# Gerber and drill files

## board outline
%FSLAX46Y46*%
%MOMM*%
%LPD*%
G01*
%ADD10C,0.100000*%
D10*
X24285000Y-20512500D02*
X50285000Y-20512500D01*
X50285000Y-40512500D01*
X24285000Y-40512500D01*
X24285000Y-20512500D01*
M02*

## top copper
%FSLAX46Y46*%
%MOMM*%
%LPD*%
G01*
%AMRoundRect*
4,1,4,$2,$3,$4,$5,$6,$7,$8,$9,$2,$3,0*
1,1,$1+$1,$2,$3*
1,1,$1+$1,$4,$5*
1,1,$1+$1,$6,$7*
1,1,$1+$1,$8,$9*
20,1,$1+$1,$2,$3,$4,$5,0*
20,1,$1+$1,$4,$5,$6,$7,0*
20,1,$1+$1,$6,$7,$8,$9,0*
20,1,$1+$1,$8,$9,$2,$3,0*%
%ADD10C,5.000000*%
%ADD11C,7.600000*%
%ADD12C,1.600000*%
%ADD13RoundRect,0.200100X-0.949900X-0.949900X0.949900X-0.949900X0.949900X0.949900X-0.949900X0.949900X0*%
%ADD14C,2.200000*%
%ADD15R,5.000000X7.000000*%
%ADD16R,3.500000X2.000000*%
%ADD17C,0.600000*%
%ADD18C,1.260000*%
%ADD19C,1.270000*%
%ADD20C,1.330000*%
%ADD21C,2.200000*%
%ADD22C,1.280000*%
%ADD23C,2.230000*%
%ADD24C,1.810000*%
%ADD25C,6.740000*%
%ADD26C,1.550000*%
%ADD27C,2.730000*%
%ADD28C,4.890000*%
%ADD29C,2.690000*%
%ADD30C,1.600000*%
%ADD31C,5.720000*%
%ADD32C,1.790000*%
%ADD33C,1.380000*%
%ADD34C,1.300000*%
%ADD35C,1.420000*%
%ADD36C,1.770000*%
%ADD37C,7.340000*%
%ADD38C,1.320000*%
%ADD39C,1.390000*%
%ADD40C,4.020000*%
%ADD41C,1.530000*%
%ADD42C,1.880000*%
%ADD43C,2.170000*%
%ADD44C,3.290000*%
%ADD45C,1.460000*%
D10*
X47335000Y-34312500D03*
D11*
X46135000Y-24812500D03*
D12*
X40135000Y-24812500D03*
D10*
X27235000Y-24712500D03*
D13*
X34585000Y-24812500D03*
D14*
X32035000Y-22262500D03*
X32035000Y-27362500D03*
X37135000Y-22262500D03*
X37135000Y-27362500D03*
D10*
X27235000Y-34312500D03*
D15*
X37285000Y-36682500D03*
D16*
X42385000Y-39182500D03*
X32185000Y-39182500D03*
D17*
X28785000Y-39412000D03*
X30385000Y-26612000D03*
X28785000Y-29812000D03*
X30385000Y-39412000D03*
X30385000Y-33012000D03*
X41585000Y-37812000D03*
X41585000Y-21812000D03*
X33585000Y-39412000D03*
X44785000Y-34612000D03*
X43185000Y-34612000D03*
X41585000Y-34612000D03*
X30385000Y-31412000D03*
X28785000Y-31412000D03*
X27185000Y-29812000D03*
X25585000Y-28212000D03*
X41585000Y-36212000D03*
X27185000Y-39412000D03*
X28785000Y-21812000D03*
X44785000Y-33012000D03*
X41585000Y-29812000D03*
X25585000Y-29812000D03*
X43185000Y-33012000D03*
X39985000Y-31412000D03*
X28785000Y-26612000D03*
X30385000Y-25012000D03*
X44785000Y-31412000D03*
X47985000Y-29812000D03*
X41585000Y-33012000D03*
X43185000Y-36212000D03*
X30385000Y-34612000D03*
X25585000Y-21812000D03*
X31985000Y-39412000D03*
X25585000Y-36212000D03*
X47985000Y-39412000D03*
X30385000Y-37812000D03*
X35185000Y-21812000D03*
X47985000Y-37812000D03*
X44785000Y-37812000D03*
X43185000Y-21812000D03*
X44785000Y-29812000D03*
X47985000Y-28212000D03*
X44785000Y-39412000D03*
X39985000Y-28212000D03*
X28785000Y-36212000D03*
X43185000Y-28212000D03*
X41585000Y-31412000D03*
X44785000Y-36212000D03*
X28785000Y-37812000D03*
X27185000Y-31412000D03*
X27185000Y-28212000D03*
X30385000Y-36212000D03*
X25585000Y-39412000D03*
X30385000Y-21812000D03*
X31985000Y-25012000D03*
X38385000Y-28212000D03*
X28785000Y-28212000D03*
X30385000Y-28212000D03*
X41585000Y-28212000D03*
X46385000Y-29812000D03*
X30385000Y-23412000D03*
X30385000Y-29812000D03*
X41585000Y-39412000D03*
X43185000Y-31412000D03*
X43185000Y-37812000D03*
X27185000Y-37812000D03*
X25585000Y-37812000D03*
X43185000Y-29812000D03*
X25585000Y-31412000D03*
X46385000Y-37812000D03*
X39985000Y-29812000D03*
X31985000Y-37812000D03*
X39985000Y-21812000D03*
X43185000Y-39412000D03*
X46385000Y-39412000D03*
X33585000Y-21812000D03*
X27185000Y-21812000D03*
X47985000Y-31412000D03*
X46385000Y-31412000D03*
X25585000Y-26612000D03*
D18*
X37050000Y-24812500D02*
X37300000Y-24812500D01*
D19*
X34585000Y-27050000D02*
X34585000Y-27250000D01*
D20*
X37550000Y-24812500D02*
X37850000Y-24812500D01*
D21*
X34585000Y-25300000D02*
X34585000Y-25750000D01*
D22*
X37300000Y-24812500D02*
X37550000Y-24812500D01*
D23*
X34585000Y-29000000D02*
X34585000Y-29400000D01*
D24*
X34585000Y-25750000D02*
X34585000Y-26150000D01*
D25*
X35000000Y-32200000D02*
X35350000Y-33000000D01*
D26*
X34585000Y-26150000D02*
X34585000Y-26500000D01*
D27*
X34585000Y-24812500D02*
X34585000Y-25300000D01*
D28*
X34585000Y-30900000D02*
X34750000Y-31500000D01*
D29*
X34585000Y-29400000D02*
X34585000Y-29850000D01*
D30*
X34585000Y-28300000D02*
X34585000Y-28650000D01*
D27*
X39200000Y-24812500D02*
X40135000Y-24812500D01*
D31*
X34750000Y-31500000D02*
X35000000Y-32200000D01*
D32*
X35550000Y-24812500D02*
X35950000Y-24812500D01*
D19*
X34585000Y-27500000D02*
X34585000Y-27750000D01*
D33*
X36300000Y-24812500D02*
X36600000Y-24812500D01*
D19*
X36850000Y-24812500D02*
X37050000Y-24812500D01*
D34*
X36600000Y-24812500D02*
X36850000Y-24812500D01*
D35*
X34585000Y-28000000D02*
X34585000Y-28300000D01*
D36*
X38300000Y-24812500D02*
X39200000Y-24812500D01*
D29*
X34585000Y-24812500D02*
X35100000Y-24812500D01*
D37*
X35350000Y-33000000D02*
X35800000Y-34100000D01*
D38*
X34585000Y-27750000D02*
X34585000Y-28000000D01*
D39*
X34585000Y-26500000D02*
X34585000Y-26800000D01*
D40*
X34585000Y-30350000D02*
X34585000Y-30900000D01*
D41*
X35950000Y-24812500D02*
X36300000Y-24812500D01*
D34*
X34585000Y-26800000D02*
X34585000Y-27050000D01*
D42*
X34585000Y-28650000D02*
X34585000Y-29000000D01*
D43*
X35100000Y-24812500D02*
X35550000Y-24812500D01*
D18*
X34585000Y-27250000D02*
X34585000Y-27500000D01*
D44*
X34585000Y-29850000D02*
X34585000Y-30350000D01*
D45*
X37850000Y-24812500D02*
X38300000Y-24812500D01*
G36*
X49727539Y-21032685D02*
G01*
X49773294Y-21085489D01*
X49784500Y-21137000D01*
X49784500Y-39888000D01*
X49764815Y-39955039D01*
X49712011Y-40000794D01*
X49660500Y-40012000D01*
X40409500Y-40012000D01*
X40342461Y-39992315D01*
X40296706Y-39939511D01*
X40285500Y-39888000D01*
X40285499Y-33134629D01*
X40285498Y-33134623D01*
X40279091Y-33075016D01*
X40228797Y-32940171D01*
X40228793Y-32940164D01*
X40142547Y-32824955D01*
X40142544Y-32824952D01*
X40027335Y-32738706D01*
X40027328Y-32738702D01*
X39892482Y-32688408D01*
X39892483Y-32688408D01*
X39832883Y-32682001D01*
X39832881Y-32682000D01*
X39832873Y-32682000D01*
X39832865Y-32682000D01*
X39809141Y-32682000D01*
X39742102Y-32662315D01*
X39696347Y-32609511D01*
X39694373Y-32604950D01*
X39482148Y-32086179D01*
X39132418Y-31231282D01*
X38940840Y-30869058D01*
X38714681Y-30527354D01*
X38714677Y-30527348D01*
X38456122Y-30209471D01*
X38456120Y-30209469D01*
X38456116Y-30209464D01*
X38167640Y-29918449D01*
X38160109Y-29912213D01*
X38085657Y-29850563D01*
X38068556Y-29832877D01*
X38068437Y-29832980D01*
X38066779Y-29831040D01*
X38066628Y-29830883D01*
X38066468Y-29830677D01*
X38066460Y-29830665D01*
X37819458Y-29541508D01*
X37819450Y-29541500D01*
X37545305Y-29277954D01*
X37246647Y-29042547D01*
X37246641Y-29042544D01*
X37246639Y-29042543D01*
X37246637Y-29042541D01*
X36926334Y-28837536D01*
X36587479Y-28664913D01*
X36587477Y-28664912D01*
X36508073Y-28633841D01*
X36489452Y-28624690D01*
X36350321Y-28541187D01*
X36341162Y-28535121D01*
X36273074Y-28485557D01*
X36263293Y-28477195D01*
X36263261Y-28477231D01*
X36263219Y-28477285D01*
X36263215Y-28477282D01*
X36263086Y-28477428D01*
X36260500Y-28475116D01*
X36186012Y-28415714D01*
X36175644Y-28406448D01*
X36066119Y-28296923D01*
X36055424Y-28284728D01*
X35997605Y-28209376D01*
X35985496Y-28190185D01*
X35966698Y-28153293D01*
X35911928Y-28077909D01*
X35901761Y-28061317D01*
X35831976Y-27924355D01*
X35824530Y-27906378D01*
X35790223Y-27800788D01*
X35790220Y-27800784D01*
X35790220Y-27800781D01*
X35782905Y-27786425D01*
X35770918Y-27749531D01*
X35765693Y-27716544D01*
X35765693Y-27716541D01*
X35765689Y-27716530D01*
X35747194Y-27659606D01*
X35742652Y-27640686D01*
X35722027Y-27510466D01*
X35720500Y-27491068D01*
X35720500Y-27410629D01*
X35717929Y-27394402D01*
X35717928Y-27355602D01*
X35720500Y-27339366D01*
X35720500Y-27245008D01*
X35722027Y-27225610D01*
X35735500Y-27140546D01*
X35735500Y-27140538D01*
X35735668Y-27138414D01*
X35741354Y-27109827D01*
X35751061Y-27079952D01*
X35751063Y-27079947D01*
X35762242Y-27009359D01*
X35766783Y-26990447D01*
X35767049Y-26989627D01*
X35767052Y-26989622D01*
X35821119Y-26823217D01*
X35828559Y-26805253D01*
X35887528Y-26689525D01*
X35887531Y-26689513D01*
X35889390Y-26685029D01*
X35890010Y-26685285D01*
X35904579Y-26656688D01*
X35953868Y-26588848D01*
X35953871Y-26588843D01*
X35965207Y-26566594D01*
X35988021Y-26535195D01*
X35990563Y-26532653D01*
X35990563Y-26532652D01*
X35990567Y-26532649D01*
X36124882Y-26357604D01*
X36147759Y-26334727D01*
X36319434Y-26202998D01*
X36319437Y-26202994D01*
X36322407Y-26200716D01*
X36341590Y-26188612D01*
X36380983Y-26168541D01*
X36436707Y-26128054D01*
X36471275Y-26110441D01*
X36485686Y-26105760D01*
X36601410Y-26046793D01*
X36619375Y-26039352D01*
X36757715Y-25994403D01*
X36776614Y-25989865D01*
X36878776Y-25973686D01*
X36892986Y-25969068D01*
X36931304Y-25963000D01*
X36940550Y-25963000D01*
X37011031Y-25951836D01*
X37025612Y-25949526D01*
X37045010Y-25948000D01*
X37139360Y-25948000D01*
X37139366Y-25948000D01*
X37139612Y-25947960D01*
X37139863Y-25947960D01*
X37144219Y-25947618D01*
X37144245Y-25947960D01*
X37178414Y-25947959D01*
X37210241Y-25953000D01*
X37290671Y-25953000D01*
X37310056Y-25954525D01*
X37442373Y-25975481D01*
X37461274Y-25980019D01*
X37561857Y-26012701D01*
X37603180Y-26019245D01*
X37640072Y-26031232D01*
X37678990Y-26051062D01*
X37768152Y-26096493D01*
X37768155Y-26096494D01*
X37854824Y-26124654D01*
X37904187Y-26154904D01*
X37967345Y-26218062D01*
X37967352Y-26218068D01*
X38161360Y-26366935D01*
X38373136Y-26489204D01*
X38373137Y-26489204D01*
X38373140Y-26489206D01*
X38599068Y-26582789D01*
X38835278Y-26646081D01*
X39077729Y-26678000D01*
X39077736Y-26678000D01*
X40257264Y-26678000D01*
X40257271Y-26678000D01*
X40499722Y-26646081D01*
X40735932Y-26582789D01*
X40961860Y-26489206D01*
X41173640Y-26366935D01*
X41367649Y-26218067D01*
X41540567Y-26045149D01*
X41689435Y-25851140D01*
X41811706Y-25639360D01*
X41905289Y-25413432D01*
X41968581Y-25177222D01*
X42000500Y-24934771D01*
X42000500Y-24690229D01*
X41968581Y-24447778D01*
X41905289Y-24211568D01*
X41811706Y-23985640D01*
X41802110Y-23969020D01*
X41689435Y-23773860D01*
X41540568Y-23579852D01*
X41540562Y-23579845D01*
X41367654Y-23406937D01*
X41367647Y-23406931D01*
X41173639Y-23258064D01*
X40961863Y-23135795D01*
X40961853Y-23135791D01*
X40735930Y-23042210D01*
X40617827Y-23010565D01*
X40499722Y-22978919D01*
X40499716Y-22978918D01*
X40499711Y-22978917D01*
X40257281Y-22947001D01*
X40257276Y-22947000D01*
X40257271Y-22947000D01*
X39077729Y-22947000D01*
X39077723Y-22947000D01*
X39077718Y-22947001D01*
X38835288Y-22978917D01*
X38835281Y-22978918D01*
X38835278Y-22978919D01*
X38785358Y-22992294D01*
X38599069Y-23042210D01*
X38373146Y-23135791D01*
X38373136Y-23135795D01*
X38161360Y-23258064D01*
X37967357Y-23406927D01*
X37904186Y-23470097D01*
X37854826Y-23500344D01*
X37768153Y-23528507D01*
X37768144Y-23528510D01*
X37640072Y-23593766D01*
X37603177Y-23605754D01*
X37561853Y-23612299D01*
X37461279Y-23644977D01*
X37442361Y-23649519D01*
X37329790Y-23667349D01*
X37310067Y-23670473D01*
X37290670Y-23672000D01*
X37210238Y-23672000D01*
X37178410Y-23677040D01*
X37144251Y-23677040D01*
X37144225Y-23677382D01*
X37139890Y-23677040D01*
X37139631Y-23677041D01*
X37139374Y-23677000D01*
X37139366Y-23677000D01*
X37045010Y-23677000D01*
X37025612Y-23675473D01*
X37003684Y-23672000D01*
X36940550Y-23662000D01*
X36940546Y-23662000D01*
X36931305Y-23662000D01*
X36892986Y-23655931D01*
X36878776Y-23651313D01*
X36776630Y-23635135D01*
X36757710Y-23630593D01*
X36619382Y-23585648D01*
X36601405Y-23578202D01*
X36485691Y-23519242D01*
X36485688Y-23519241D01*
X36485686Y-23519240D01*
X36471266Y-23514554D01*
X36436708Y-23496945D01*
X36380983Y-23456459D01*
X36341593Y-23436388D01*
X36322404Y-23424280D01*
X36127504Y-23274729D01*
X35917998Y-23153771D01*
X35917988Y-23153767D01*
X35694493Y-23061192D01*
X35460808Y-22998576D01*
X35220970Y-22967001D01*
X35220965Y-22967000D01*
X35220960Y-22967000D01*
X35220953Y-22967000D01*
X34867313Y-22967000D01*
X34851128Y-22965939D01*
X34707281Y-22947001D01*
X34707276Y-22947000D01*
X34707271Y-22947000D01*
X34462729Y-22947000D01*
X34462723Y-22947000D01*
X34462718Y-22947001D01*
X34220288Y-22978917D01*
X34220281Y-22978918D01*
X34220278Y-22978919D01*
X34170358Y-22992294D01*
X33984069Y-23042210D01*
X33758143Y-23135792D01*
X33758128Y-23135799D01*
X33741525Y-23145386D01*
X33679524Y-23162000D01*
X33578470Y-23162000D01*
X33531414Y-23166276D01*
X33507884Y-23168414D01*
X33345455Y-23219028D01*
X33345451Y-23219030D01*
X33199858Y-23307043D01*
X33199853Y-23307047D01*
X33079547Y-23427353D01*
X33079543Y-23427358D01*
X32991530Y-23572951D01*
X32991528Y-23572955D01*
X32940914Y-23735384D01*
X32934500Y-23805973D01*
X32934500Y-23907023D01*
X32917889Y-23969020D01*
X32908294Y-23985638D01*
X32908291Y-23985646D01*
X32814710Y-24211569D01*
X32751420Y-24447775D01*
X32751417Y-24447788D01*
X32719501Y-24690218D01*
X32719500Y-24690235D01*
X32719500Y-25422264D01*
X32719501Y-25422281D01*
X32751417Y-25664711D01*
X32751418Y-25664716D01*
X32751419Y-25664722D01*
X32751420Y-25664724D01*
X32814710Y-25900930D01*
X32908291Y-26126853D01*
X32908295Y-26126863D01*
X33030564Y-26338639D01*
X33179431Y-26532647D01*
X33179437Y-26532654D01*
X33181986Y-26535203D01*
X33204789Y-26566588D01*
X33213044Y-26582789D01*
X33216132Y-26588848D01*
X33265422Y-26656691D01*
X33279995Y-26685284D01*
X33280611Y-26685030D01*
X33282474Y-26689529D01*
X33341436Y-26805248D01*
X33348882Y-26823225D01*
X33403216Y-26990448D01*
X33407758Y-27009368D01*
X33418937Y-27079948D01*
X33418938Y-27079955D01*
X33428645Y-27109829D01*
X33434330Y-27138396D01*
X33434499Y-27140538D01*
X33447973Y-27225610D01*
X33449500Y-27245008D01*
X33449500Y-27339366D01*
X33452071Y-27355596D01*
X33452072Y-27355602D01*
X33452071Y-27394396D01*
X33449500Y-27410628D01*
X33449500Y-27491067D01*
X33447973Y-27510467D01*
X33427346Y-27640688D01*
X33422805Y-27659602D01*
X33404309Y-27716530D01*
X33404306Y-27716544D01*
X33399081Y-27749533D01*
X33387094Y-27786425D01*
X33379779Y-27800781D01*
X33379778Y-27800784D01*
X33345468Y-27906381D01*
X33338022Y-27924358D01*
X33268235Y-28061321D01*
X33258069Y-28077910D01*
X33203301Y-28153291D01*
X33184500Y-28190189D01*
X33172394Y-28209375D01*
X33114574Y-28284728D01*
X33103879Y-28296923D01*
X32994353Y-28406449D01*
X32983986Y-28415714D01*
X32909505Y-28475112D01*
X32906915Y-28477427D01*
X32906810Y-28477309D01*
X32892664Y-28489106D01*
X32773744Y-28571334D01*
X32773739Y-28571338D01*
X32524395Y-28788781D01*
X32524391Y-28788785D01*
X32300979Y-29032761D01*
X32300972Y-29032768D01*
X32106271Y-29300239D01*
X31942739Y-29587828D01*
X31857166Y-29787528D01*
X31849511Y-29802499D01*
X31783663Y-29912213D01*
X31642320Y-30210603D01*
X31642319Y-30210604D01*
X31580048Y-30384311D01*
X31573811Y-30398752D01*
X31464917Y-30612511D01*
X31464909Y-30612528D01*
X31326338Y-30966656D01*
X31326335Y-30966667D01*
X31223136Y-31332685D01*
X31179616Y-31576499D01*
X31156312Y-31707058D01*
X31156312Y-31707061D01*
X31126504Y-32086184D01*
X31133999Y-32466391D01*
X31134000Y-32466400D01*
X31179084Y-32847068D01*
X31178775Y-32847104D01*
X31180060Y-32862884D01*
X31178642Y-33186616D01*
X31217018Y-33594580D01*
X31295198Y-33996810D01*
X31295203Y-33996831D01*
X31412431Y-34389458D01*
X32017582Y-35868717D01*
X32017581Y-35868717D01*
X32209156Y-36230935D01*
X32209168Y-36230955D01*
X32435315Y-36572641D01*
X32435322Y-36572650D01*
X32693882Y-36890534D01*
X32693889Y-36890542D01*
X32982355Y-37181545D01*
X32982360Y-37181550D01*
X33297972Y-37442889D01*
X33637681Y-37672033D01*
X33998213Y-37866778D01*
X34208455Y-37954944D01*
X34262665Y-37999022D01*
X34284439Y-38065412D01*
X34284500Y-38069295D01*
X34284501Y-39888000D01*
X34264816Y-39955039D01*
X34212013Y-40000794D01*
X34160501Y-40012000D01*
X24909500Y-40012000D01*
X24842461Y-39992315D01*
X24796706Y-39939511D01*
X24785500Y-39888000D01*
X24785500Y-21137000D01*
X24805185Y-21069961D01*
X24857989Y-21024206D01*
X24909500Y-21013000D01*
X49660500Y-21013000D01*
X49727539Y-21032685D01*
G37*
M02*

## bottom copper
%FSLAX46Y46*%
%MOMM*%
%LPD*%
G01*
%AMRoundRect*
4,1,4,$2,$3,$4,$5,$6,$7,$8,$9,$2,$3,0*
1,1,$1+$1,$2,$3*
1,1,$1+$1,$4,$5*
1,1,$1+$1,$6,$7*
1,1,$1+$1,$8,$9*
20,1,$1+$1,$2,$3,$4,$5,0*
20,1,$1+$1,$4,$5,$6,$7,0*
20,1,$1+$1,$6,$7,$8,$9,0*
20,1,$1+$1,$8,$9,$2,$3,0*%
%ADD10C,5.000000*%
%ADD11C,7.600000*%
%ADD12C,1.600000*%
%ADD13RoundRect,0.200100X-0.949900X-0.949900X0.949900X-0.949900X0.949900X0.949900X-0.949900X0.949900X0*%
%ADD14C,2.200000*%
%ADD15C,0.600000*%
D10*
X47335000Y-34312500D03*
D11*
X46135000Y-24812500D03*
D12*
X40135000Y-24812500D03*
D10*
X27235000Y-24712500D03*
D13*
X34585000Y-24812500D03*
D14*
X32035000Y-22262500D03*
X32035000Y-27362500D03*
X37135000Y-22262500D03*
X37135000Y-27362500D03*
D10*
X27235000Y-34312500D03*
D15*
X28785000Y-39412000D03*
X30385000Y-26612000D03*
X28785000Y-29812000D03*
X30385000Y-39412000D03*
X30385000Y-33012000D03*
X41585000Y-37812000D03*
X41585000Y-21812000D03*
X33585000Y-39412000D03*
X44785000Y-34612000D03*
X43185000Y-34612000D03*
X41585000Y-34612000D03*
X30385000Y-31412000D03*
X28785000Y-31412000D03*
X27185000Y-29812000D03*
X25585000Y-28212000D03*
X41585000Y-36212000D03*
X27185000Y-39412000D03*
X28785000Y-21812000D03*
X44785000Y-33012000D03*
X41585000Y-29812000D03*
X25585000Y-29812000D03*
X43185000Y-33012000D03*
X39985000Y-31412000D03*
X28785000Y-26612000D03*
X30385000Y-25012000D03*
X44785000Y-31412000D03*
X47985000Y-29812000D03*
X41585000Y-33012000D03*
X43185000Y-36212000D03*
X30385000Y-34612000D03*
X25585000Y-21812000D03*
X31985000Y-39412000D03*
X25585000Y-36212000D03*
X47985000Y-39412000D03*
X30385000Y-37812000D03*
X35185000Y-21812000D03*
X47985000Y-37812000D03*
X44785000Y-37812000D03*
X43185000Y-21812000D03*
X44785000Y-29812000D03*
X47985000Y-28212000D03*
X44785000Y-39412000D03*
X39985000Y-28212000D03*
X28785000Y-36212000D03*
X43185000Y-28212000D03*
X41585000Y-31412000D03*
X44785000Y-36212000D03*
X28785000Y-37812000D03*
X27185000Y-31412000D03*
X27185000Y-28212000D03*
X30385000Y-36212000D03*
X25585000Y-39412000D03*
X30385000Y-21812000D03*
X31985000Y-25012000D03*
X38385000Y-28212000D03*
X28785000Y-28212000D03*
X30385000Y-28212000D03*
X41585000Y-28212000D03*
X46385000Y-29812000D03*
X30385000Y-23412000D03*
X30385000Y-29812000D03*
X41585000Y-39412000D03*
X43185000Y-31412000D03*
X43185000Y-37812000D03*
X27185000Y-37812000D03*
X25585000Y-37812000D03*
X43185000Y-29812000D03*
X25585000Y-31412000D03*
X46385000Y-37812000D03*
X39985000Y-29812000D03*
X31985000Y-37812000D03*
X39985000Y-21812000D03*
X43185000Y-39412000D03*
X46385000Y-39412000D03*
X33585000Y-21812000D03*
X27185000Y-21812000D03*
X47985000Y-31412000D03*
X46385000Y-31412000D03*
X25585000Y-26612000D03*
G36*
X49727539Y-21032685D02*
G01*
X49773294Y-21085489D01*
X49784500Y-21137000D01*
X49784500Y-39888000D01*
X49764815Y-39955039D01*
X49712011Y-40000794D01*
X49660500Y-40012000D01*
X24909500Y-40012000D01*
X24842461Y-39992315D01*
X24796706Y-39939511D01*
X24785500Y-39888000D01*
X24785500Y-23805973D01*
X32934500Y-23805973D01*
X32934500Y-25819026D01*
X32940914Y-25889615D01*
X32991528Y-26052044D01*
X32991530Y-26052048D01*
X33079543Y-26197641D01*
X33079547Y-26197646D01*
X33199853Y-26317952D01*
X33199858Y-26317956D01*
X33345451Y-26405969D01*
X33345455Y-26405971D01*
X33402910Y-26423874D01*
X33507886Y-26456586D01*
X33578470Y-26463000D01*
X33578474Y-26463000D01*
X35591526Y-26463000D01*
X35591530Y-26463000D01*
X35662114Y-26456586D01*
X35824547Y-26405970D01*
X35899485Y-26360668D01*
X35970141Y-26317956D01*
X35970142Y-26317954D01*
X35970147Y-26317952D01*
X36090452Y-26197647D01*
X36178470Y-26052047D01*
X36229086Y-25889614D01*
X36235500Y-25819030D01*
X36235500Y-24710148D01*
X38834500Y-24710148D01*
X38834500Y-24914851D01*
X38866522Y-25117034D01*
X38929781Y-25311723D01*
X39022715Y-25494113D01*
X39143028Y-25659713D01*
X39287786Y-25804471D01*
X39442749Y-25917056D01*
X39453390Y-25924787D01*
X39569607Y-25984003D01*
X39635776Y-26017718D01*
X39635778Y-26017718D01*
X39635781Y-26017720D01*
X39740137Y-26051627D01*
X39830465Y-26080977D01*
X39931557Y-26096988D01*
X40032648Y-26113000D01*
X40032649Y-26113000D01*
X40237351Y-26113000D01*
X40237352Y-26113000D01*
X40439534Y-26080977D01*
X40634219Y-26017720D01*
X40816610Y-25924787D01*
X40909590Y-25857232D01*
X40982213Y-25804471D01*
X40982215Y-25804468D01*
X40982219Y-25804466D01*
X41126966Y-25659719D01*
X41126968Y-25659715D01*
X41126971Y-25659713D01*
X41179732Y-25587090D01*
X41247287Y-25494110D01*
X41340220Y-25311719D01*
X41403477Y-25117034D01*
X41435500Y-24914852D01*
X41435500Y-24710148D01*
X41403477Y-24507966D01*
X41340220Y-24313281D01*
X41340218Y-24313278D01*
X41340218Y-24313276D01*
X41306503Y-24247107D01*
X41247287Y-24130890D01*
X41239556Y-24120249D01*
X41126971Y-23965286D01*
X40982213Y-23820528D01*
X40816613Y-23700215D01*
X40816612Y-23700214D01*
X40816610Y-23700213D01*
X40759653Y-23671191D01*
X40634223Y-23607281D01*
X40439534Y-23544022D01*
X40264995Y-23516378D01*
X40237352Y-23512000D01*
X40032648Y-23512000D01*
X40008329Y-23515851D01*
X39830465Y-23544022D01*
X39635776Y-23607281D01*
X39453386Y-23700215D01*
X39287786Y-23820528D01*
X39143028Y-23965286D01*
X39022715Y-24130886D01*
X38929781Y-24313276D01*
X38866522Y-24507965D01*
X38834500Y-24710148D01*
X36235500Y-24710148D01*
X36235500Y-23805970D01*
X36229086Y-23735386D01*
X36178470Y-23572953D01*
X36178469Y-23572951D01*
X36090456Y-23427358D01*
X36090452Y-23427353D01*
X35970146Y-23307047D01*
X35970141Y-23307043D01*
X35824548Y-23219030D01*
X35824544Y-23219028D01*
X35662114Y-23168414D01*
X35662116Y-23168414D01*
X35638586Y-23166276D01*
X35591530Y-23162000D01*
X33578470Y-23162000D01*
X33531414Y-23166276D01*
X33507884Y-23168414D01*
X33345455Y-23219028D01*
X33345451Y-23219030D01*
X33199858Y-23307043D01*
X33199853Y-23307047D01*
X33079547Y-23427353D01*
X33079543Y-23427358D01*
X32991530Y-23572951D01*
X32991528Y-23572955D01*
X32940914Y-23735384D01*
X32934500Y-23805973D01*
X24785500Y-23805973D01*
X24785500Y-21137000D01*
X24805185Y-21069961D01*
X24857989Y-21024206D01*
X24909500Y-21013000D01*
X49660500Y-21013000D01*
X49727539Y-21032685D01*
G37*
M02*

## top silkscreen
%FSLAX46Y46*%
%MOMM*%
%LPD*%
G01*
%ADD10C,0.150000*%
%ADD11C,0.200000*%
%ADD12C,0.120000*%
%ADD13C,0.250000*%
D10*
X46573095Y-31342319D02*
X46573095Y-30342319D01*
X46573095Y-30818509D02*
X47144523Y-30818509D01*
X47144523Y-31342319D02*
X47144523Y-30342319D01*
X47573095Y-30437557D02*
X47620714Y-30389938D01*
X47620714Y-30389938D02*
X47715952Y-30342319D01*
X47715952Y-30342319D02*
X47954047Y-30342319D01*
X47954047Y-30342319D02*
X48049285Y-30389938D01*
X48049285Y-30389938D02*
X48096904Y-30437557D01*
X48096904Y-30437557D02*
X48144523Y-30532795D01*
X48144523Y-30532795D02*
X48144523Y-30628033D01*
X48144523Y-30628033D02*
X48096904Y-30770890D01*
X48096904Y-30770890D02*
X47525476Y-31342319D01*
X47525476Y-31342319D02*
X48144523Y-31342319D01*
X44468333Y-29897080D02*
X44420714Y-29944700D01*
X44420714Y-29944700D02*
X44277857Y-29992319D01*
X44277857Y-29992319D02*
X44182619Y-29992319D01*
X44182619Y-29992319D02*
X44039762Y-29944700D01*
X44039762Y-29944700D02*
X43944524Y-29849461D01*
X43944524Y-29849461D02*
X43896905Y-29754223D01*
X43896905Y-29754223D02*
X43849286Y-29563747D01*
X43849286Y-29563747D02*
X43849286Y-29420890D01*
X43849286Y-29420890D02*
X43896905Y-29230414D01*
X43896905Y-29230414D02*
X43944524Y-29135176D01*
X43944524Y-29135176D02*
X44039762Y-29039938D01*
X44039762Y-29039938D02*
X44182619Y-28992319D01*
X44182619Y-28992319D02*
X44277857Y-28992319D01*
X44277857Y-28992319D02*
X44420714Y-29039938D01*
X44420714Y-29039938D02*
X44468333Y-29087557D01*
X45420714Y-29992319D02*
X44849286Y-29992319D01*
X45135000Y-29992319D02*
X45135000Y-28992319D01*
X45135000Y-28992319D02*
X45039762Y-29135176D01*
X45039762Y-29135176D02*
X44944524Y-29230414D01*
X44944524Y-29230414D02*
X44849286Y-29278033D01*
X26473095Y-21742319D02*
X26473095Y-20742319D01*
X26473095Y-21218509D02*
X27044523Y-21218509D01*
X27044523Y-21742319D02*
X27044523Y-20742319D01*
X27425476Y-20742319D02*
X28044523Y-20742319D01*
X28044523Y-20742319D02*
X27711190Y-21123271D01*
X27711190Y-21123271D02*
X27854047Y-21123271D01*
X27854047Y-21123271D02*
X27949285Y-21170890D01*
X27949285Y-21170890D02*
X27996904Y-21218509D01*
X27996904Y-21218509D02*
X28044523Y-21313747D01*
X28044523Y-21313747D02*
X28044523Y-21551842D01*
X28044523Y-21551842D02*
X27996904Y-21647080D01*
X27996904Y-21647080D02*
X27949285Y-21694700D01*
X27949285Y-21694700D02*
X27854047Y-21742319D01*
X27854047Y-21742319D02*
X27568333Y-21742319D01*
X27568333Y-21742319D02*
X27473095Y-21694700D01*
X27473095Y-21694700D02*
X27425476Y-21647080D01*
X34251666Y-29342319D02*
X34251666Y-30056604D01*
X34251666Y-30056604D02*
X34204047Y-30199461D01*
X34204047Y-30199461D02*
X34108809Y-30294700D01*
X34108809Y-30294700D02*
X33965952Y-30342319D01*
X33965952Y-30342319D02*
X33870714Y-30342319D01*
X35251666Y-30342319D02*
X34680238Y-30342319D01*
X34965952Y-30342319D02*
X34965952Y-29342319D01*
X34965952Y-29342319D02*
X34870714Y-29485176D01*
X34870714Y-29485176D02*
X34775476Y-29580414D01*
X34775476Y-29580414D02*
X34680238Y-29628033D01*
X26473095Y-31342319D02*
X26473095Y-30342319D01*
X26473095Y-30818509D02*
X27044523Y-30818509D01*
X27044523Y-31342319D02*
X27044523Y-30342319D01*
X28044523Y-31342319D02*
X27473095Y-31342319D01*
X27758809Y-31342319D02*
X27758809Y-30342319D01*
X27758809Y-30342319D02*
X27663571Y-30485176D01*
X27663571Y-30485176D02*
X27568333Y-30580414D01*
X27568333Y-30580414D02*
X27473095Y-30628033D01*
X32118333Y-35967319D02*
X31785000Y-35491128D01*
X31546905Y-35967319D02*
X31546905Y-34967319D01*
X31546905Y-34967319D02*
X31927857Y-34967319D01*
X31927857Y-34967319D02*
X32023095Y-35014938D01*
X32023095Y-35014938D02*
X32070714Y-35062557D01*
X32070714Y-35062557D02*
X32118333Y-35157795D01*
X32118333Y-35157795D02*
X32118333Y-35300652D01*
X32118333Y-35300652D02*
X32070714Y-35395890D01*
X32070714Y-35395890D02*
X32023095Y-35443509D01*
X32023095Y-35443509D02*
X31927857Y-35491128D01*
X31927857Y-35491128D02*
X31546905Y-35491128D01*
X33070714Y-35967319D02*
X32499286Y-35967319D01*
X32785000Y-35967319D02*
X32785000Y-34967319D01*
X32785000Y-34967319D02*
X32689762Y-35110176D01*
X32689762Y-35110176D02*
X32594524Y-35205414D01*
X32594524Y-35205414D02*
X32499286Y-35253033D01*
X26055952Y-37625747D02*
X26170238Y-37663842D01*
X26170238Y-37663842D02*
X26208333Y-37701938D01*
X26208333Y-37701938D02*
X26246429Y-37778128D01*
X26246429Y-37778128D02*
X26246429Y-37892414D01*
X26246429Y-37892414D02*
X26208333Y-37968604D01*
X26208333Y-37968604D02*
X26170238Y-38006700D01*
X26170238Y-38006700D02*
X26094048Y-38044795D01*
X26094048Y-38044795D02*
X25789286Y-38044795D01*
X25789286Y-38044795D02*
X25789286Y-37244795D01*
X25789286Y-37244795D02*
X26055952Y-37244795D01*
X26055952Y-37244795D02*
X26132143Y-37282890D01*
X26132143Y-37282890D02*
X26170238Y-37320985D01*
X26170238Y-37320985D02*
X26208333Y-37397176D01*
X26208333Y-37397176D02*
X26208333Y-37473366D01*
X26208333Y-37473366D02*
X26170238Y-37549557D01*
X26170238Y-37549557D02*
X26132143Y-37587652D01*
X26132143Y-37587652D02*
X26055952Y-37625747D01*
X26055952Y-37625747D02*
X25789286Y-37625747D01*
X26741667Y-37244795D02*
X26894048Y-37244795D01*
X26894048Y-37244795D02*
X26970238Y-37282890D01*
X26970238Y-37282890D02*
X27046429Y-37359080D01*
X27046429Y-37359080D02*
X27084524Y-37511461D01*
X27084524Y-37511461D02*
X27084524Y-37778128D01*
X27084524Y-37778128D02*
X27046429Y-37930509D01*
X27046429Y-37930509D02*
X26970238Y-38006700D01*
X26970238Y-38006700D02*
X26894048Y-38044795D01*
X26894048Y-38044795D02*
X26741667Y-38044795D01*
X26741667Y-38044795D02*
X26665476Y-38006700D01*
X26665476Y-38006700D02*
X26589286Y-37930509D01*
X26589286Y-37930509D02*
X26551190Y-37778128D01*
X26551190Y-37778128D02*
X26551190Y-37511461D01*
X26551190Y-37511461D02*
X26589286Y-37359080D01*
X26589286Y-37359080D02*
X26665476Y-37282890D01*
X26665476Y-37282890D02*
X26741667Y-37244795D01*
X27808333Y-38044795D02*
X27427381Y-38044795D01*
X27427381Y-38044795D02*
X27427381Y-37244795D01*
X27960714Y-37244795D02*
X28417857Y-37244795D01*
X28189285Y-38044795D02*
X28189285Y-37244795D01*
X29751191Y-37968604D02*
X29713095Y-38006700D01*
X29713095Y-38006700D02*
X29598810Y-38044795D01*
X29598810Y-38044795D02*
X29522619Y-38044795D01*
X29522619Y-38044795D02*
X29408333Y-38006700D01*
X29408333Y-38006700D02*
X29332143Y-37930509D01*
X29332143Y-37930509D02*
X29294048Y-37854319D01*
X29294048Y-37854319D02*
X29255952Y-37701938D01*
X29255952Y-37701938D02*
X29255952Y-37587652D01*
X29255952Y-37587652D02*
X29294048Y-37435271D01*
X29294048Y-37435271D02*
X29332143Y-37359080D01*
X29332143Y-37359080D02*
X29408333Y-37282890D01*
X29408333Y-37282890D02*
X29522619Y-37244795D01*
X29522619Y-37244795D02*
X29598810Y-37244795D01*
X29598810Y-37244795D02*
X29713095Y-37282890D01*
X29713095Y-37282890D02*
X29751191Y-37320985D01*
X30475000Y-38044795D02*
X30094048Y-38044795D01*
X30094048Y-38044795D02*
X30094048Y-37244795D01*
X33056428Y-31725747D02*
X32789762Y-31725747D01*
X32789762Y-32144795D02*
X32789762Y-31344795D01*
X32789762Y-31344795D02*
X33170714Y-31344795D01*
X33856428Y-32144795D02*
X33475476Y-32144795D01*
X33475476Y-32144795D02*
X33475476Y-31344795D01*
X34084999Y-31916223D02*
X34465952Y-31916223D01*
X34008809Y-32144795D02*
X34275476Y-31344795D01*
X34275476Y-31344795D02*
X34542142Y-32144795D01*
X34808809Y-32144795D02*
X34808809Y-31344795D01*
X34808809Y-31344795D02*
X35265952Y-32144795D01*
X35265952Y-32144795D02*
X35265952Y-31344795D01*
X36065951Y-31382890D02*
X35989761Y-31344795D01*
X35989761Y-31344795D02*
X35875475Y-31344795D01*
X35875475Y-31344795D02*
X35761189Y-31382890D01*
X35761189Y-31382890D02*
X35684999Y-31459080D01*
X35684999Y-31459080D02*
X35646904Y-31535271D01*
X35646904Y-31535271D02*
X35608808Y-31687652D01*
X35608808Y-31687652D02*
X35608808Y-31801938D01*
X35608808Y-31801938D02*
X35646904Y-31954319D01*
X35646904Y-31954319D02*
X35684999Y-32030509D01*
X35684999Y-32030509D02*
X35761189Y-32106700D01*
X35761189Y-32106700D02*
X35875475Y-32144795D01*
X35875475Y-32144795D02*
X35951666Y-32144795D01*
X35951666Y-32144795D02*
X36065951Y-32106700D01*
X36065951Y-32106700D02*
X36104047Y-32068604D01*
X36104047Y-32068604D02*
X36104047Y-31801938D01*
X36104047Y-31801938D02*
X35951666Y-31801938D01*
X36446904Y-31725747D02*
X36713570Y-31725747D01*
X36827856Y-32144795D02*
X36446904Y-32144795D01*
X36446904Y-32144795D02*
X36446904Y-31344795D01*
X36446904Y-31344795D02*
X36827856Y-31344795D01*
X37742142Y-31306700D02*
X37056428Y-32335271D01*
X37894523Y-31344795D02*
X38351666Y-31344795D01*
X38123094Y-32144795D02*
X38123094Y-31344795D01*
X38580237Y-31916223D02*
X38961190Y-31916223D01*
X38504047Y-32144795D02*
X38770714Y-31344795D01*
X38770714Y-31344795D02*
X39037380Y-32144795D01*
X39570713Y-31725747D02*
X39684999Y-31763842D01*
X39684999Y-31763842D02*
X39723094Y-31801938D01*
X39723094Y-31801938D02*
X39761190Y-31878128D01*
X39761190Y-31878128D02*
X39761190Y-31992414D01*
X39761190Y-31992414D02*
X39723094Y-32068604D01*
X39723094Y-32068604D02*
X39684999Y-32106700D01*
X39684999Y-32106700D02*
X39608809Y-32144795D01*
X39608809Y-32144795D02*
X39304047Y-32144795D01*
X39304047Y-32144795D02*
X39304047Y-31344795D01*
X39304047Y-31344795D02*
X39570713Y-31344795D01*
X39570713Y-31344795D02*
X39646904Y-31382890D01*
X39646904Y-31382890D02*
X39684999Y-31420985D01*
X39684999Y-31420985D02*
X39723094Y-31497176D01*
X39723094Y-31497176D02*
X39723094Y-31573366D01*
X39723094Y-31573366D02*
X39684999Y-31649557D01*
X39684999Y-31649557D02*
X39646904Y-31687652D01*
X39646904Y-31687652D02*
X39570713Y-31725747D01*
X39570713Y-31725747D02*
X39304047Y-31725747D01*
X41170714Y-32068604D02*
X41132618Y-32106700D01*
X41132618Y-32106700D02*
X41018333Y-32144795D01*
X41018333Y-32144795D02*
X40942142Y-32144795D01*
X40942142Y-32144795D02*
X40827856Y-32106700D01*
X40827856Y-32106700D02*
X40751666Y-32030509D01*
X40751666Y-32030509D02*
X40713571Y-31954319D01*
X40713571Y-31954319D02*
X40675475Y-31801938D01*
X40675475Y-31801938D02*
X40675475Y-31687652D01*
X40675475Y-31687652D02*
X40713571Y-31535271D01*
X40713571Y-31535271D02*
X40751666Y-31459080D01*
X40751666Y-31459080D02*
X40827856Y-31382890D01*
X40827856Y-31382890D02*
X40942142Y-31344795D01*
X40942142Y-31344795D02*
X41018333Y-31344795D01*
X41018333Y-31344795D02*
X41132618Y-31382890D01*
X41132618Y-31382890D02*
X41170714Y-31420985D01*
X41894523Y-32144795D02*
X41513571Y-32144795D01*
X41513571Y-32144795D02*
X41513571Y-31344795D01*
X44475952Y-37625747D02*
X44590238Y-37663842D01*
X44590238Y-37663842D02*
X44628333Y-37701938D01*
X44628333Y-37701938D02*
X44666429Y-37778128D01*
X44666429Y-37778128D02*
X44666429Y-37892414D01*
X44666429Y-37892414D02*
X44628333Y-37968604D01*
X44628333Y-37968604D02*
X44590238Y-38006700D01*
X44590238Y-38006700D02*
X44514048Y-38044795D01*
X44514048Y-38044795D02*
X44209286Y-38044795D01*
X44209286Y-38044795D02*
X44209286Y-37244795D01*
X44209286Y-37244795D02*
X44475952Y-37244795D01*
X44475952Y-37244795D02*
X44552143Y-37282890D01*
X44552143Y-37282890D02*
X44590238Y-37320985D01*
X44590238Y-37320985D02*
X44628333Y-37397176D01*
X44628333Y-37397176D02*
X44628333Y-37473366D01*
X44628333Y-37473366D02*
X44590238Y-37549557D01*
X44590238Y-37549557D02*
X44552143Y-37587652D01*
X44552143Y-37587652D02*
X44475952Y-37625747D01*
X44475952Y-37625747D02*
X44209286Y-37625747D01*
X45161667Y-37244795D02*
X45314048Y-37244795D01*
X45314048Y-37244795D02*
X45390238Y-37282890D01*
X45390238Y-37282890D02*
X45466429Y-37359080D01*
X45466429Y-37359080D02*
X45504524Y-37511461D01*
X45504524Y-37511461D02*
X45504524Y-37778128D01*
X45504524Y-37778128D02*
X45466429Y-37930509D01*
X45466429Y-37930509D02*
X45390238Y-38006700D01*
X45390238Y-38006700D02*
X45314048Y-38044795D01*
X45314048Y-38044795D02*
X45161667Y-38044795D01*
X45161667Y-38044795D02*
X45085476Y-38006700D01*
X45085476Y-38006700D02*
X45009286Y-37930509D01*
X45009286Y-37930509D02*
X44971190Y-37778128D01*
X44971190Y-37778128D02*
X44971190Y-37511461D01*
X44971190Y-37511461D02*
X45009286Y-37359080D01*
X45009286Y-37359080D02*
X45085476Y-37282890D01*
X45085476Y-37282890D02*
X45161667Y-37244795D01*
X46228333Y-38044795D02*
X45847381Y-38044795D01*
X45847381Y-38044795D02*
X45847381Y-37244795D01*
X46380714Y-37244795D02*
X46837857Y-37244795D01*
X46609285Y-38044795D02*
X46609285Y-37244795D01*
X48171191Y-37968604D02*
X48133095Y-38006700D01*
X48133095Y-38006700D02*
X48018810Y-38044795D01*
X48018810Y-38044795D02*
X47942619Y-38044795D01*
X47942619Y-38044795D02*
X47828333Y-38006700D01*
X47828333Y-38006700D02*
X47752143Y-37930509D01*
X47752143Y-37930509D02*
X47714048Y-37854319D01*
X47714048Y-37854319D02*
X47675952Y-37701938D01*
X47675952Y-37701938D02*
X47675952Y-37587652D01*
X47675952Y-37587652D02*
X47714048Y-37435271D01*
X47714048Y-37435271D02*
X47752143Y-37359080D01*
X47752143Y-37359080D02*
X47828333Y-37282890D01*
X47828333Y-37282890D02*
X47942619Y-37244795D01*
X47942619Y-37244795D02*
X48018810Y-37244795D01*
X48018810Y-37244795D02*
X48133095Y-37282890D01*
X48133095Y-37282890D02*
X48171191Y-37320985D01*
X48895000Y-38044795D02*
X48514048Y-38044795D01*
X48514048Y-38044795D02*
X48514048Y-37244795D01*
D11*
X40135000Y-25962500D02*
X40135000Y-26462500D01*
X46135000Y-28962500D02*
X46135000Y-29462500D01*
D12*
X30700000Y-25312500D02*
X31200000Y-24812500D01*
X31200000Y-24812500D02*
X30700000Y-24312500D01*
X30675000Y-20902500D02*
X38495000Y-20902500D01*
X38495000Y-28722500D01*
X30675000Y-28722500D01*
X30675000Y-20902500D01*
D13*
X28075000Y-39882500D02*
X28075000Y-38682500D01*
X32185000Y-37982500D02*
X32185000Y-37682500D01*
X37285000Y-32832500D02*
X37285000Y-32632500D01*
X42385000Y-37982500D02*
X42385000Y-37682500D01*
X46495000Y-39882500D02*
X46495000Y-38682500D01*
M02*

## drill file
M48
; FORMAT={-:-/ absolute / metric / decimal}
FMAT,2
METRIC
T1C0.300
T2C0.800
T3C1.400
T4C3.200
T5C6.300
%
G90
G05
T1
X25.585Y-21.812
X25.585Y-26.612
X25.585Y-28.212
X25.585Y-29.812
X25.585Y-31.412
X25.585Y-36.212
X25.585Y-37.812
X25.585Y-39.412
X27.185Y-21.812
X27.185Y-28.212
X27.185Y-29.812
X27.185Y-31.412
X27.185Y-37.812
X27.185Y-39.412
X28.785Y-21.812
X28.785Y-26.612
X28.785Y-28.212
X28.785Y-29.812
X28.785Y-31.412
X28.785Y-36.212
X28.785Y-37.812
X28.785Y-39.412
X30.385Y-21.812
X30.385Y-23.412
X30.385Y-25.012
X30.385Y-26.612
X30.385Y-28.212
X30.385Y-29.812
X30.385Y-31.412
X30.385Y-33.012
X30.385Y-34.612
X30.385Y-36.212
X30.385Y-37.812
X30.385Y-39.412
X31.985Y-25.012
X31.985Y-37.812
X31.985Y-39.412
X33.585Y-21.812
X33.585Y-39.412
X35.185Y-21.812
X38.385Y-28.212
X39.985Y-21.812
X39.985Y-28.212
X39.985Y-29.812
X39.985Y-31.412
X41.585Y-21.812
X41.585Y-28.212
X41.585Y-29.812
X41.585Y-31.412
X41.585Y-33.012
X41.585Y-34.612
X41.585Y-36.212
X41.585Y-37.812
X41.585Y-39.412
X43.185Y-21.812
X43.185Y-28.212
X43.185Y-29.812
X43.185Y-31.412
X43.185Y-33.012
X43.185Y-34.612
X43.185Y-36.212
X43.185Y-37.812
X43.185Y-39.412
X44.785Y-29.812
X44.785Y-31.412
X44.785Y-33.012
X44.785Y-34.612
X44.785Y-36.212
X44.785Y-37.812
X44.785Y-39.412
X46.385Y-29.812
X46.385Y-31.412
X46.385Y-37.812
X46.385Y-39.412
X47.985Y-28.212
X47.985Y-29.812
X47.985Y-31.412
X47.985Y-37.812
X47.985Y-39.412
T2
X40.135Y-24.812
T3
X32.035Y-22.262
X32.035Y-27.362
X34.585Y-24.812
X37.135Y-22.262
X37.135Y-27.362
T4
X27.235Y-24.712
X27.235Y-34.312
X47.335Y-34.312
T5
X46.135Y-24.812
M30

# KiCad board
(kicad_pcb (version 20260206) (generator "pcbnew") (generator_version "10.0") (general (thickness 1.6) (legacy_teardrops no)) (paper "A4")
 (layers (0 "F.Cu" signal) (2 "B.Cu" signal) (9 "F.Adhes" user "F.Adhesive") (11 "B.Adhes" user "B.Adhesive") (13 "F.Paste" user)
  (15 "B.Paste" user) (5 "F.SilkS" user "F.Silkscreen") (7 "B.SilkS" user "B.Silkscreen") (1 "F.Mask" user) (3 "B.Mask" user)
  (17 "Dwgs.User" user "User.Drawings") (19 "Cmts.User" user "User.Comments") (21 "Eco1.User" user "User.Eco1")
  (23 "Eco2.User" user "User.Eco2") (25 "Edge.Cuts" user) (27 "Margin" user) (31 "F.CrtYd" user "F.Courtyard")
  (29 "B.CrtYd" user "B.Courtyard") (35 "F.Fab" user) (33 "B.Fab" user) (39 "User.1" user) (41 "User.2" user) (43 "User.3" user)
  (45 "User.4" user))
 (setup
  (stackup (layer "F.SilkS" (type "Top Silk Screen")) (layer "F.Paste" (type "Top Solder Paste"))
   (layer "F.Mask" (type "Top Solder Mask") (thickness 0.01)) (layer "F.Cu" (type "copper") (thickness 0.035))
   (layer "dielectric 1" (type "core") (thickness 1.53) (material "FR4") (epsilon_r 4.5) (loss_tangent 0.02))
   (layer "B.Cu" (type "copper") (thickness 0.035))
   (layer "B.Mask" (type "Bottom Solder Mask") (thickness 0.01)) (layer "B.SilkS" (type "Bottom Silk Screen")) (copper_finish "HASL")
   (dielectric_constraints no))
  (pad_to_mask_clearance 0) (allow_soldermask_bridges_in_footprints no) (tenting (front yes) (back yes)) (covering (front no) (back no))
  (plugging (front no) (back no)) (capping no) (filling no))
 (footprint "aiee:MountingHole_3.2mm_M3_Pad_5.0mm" (layer "F.Cu") (at 47.335 34.3125)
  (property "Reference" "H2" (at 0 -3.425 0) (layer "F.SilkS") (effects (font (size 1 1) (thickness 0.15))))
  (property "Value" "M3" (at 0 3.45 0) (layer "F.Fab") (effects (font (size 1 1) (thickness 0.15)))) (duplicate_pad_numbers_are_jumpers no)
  (pad "1" thru_hole circle (at 0 0) (size 5 5) (drill 3.2) (layers "*.Cu" "*.Mask") (remove_unused_layers no) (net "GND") (zone_connect 2)))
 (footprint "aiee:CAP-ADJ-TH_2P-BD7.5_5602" (layer "F.Cu") (at 46.135 24.8125 180)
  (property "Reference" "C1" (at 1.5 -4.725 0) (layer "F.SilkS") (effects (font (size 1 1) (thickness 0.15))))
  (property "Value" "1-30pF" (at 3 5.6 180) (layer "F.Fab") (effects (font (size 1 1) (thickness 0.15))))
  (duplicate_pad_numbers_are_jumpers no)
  (fp_line (start 6 -1.15) (end 6 -1.65) (stroke (width 0.2) (type solid)) (layer "F.SilkS"))
  (fp_line (start 0 -4.15) (end 0 -4.65) (stroke (width 0.2) (type solid)) (layer "F.SilkS"))
  (pad "1" thru_hole circle (at 0 0 180) (size 7.6 7.6) (drill 6.3) (layers "*.Cu" "*.Mask") (remove_unused_layers no) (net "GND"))
  (pad "2" thru_hole circle (at 6 0 180) (size 1.6 1.6) (drill 0.8) (layers "*.Cu" "*.Mask") (remove_unused_layers no) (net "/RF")))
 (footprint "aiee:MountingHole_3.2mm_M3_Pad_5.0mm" (layer "F.Cu") (at 27.235 24.7125)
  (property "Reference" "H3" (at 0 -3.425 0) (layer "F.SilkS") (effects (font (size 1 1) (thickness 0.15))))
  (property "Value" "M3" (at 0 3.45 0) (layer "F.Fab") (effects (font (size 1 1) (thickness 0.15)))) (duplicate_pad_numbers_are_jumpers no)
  (pad "1" thru_hole circle (at 0 0) (size 5 5) (drill 3.2) (layers "*.Cu" "*.Mask") (remove_unused_layers no) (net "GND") (zone_connect 2)))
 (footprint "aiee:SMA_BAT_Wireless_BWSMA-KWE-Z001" (layer "F.Cu") (at 34.585 24.8125)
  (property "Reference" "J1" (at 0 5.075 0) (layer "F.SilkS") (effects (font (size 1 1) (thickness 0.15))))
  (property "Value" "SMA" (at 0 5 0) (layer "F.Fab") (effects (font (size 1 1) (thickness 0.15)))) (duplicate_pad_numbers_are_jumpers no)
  (fp_line (start -3.885 0.5) (end -3.385 0) (stroke (width 0.12) (type solid)) (layer "F.SilkS"))
  (fp_line (start -3.385 0) (end -3.885 -0.5) (stroke (width 0.12) (type solid)) (layer "F.SilkS"))
  (fp_rect (start -3.91 -3.91) (end 3.91 3.91) (stroke (width 0.12) (type default)) (fill no) (layer "F.SilkS"))
  (pad "1" thru_hole roundrect (at 0 0) (size 2.3 2.3) (drill 1.4) (layers "*.Cu" "*.Mask") (remove_unused_layers yes) (keep_end_layers yes)
   (zone_layer_connections) (roundrect_rratio 0.087) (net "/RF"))
  (pad "2" thru_hole circle (at -2.55 -2.55) (size 2.2 2.2) (drill 1.4) (layers "*.Cu" "*.Mask") (remove_unused_layers yes)
   (keep_end_layers yes) (zone_layer_connections) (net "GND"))
  (pad "2" thru_hole circle (at -2.55 2.55) (size 2.2 2.2) (drill 1.4) (layers "*.Cu" "*.Mask") (remove_unused_layers yes)
   (keep_end_layers yes) (zone_layer_connections) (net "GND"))
  (pad "2" thru_hole circle (at 2.55 -2.55) (size 2.2 2.2) (drill 1.4) (layers "*.Cu" "*.Mask") (remove_unused_layers yes)
   (keep_end_layers yes) (zone_layer_connections) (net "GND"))
  (pad "2" thru_hole circle (at 2.55 2.55) (size 2.2 2.2) (drill 1.4) (layers "*.Cu" "*.Mask") (remove_unused_layers yes)
   (keep_end_layers yes) (zone_layer_connections) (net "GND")))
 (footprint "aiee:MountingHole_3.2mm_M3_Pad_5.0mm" (layer "F.Cu") (at 27.235 34.3125)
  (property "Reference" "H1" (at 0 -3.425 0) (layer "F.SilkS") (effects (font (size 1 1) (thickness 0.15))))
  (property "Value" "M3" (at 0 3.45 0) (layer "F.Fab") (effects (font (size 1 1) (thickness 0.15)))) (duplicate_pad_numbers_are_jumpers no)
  (pad "1" thru_hole circle (at 0 0) (size 5 5) (drill 3.2) (layers "*.Cu" "*.Mask") (remove_unused_layers no) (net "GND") (zone_connect 2)))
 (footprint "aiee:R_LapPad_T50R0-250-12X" (layer "F.Cu") (at 37.285 40.1825 180)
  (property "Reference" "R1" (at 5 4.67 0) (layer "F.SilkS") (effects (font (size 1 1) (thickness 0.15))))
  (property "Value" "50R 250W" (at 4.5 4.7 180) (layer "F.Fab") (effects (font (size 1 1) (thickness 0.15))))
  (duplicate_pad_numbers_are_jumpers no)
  (fp_line (start 9.21 0.3) (end 9.21 1.5) (stroke (width 0.25) (type solid)) (layer "F.SilkS"))
  (fp_line (start 5.1 2.2) (end 5.1 2.5) (stroke (width 0.25) (type solid)) (layer "F.SilkS"))
  (fp_line (start 0 7.35) (end 0 7.55) (stroke (width 0.25) (type solid)) (layer "F.SilkS"))
  (fp_line (start -5.1 2.2) (end -5.1 2.5) (stroke (width 0.25) (type solid)) (layer "F.SilkS"))
  (fp_line (start -9.21 0.3) (end -9.21 1.5) (stroke (width 0.25) (type solid)) (layer "F.SilkS"))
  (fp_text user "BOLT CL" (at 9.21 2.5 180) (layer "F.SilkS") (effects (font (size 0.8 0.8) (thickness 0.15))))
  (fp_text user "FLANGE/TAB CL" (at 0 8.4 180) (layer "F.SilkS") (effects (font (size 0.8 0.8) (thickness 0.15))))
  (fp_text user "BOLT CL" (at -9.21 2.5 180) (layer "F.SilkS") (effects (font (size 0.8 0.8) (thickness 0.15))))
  (pad "1" smd rect (at 0 3.5 180) (size 5 7) (layers "F.Cu" "F.Mask" "F.Paste") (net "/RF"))
  (pad "2" smd rect (at -5.1 1 180) (size 3.5 2) (layers "F.Cu" "F.Mask" "F.Paste") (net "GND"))
  (pad "2" smd rect (at 5.1 1 180) (size 3.5 2) (layers "F.Cu" "F.Mask" "F.Paste") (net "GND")))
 (gr_rect (start 24.285 20.5125) (end 50.285 40.5125) (stroke (width 0.1) (type default)) (fill no) (layer "Edge.Cuts"))
 (via (at 28.785 39.412) (size 0.6) (drill 0.3) (layers "F.Cu" "B.Cu") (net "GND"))
 (via (at 30.385 26.612) (size 0.6) (drill 0.3) (layers "F.Cu" "B.Cu") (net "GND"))
 (via (at 28.785 29.812) (size 0.6) (drill 0.3) (layers "F.Cu" "B.Cu") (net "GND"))
 (via (at 30.385 39.412) (size 0.6) (drill 0.3) (layers "F.Cu" "B.Cu") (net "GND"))
 (via (at 30.385 33.012) (size 0.6) (drill 0.3) (layers "F.Cu" "B.Cu") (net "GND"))
 (via (at 41.585 37.812) (size 0.6) (drill 0.3) (layers "F.Cu" "B.Cu") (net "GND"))
 (via (at 41.585 21.812) (size 0.6) (drill 0.3) (layers "F.Cu" "B.Cu") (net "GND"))
 (via (at 33.585 39.412) (size 0.6) (drill 0.3) (layers "F.Cu" "B.Cu") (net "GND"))
 (via (at 44.785 34.612) (size 0.6) (drill 0.3) (layers "F.Cu" "B.Cu") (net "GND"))
 (via (at 43.185 34.612) (size 0.6) (drill 0.3) (layers "F.Cu" "B.Cu") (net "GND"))
 (via (at 41.585 34.612) (size 0.6) (drill 0.3) (layers "F.Cu" "B.Cu") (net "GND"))
 (via (at 30.385 31.412) (size 0.6) (drill 0.3) (layers "F.Cu" "B.Cu") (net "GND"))
 (via (at 28.785 31.412) (size 0.6) (drill 0.3) (layers "F.Cu" "B.Cu") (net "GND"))
 (via (at 27.185 29.812) (size 0.6) (drill 0.3) (layers "F.Cu" "B.Cu") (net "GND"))
 (via (at 25.585 28.212) (size 0.6) (drill 0.3) (layers "F.Cu" "B.Cu") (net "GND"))
 (via (at 41.585 36.212) (size 0.6) (drill 0.3) (layers "F.Cu" "B.Cu") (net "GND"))
 (via (at 27.185 39.412) (size 0.6) (drill 0.3) (layers "F.Cu" "B.Cu") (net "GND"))
 (via (at 28.785 21.812) (size 0.6) (drill 0.3) (layers "F.Cu" "B.Cu") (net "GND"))
 (via (at 44.785 33.012) (size 0.6) (drill 0.3) (layers "F.Cu" "B.Cu") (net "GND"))
 (via (at 41.585 29.812) (size 0.6) (drill 0.3) (layers "F.Cu" "B.Cu") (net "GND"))
 (via (at 25.585 29.812) (size 0.6) (drill 0.3) (layers "F.Cu" "B.Cu") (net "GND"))
 (via (at 43.185 33.012) (size 0.6) (drill 0.3) (layers "F.Cu" "B.Cu") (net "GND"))
 (via (at 39.985 31.412) (size 0.6) (drill 0.3) (layers "F.Cu" "B.Cu") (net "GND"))
 (via (at 28.785 26.612) (size 0.6) (drill 0.3) (layers "F.Cu" "B.Cu") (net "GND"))
 (via (at 30.385 25.012) (size 0.6) (drill 0.3) (layers "F.Cu" "B.Cu") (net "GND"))
 (via (at 44.785 31.412) (size 0.6) (drill 0.3) (layers "F.Cu" "B.Cu") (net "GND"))
 (via (at 47.985 29.812) (size 0.6) (drill 0.3) (layers "F.Cu" "B.Cu") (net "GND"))
 (via (at 41.585 33.012) (size 0.6) (drill 0.3) (layers "F.Cu" "B.Cu") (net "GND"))
 (via (at 43.185 36.212) (size 0.6) (drill 0.3) (layers "F.Cu" "B.Cu") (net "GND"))
 (via (at 30.385 34.612) (size 0.6) (drill 0.3) (layers "F.Cu" "B.Cu") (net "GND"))
 (via (at 25.585 21.812) (size 0.6) (drill 0.3) (layers "F.Cu" "B.Cu") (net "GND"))
 (via (at 31.985 39.412) (size 0.6) (drill 0.3) (layers "F.Cu" "B.Cu") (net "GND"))
 (via (at 25.585 36.212) (size 0.6) (drill 0.3) (layers "F.Cu" "B.Cu") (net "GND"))
 (via (at 47.985 39.412) (size 0.6) (drill 0.3) (layers "F.Cu" "B.Cu") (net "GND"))
 (via (at 30.385 37.812) (size 0.6) (drill 0.3) (layers "F.Cu" "B.Cu") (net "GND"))
 (via (at 35.185 21.812) (size 0.6) (drill 0.3) (layers "F.Cu" "B.Cu") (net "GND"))
 (via (at 47.985 37.812) (size 0.6) (drill 0.3) (layers "F.Cu" "B.Cu") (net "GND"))
 (via (at 44.785 37.812) (size 0.6) (drill 0.3) (layers "F.Cu" "B.Cu") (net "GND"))
 (via (at 43.185 21.812) (size 0.6) (drill 0.3) (layers "F.Cu" "B.Cu") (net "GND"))
 (via (at 44.785 29.812) (size 0.6) (drill 0.3) (layers "F.Cu" "B.Cu") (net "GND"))
 (via (at 47.985 28.212) (size 0.6) (drill 0.3) (layers "F.Cu" "B.Cu") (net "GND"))
 (via (at 44.785 39.412) (size 0.6) (drill 0.3) (layers "F.Cu" "B.Cu") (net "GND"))
 (via (at 39.985 28.212) (size 0.6) (drill 0.3) (layers "F.Cu" "B.Cu") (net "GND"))
 (via (at 28.785 36.212) (size 0.6) (drill 0.3) (layers "F.Cu" "B.Cu") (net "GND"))
 (via (at 43.185 28.212) (size 0.6) (drill 0.3) (layers "F.Cu" "B.Cu") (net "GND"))
 (via (at 41.585 31.412) (size 0.6) (drill 0.3) (layers "F.Cu" "B.Cu") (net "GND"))
 (via (at 44.785 36.212) (size 0.6) (drill 0.3) (layers "F.Cu" "B.Cu") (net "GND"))
 (via (at 28.785 37.812) (size 0.6) (drill 0.3) (layers "F.Cu" "B.Cu") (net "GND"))
 (via (at 27.185 31.412) (size 0.6) (drill 0.3) (layers "F.Cu" "B.Cu") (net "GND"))
 (via (at 27.185 28.212) (size 0.6) (drill 0.3) (layers "F.Cu" "B.Cu") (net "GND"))
 (via (at 30.385 36.212) (size 0.6) (drill 0.3) (layers "F.Cu" "B.Cu") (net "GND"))
 (via (at 25.585 39.412) (size 0.6) (drill 0.3) (layers "F.Cu" "B.Cu") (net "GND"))
 (via (at 30.385 21.812) (size 0.6) (drill 0.3) (layers "F.Cu" "B.Cu") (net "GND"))
 (via (at 31.985 25.012) (size 0.6) (drill 0.3) (layers "F.Cu" "B.Cu") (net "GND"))
 (via (at 38.385 28.212) (size 0.6) (drill 0.3) (layers "F.Cu" "B.Cu") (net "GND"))
 (via (at 28.785 28.212) (size 0.6) (drill 0.3) (layers "F.Cu" "B.Cu") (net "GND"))
 (via (at 30.385 28.212) (size 0.6) (drill 0.3) (layers "F.Cu" "B.Cu") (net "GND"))
 (via (at 41.585 28.212) (size 0.6) (drill 0.3) (layers "F.Cu" "B.Cu") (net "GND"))
 (via (at 46.385 29.812) (size 0.6) (drill 0.3) (layers "F.Cu" "B.Cu") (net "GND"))
 (via (at 30.385 23.412) (size 0.6) (drill 0.3) (layers "F.Cu" "B.Cu") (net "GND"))
 (via (at 30.385 29.812) (size 0.6) (drill 0.3) (layers "F.Cu" "B.Cu") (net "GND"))
 (via (at 41.585 39.412) (size 0.6) (drill 0.3) (layers "F.Cu" "B.Cu") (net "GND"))
 (via (at 43.185 31.412) (size 0.6) (drill 0.3) (layers "F.Cu" "B.Cu") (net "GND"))
 (via (at 43.185 37.812) (size 0.6) (drill 0.3) (layers "F.Cu" "B.Cu") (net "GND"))
 (via (at 27.185 37.812) (size 0.6) (drill 0.3) (layers "F.Cu" "B.Cu") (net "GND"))
 (via (at 25.585 37.812) (size 0.6) (drill 0.3) (layers "F.Cu" "B.Cu") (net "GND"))
 (via (at 43.185 29.812) (size 0.6) (drill 0.3) (layers "F.Cu" "B.Cu") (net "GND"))
 (via (at 25.585 31.412) (size 0.6) (drill 0.3) (layers "F.Cu" "B.Cu") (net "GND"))
 (via (at 46.385 37.812) (size 0.6) (drill 0.3) (layers "F.Cu" "B.Cu") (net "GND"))
 (via (at 39.985 29.812) (size 0.6) (drill 0.3) (layers "F.Cu" "B.Cu") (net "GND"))
 (via (at 31.985 37.812) (size 0.6) (drill 0.3) (layers "F.Cu" "B.Cu") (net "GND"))
 (via (at 39.985 21.812) (size 0.6) (drill 0.3) (layers "F.Cu" "B.Cu") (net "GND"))
 (via (at 43.185 39.412) (size 0.6) (drill 0.3) (layers "F.Cu" "B.Cu") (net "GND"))
 (via (at 46.385 39.412) (size 0.6) (drill 0.3) (layers "F.Cu" "B.Cu") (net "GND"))
 (via (at 33.585 21.812) (size 0.6) (drill 0.3) (layers "F.Cu" "B.Cu") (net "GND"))
 (via (at 27.185 21.812) (size 0.6) (drill 0.3) (layers "F.Cu" "B.Cu") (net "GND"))
 (via (at 47.985 31.412) (size 0.6) (drill 0.3) (layers "F.Cu" "B.Cu") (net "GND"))
 (via (at 46.385 31.412) (size 0.6) (drill 0.3) (layers "F.Cu" "B.Cu") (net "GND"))
 (via (at 25.585 26.612) (size 0.6) (drill 0.3) (layers "F.Cu" "B.Cu") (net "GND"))
 (segment (start 37.05 24.8125) (end 37.3 24.8125) (width 1.26) (layer "F.Cu") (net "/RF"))
 (segment (start 34.585 27.05) (end 34.585 27.25) (width 1.27) (layer "F.Cu") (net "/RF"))
 (segment (start 37.55 24.8125) (end 37.85 24.8125) (width 1.33) (layer "F.Cu") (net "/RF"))
 (segment (start 34.585 25.3) (end 34.585 25.75) (width 2.2) (layer "F.Cu") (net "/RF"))
 (segment (start 37.3 24.8125) (end 37.55 24.8125) (width 1.28) (layer "F.Cu") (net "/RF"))
 (segment (start 34.585 29) (end 34.585 29.4) (width 2.23) (layer "F.Cu") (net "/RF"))
 (segment (start 34.585 25.75) (end 34.585 26.15) (width 1.81) (layer "F.Cu") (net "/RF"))
 (segment (start 35 32.2) (end 35.35 33) (width 6.74) (layer "F.Cu") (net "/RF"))
 (segment (start 34.585 26.15) (end 34.585 26.5) (width 1.55) (layer "F.Cu") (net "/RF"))
 (segment (start 34.585 24.8125) (end 34.585 25.3) (width 2.73) (layer "F.Cu") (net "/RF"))
 (segment (start 34.585 30.9) (end 34.75 31.5) (width 4.89) (layer "F.Cu") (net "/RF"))
 (segment (start 34.585 29.4) (end 34.585 29.85) (width 2.69) (layer "F.Cu") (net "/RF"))
 (segment (start 34.585 28.3) (end 34.585 28.65) (width 1.6) (layer "F.Cu") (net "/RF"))
 (segment (start 39.2 24.8125) (end 40.135 24.8125) (width 2.73) (layer "F.Cu") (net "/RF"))
 (segment (start 34.75 31.5) (end 35 32.2) (width 5.72) (layer "F.Cu") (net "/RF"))
 (segment (start 35.55 24.8125) (end 35.95 24.8125) (width 1.79) (layer "F.Cu") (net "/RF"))
 (segment (start 34.585 27.5) (end 34.585 27.75) (width 1.27) (layer "F.Cu") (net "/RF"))
 (segment (start 36.3 24.8125) (end 36.6 24.8125) (width 1.38) (layer "F.Cu") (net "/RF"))
 (segment (start 36.85 24.8125) (end 37.05 24.8125) (width 1.27) (layer "F.Cu") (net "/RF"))
 (segment (start 36.6 24.8125) (end 36.85 24.8125) (width 1.3) (layer "F.Cu") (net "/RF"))
 (segment (start 34.585 28) (end 34.585 28.3) (width 1.42) (layer "F.Cu") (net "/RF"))
 (segment (start 38.3 24.8125) (end 39.2 24.8125) (width 1.77) (layer "F.Cu") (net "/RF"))
 (segment (start 34.585 24.8125) (end 35.1 24.8125) (width 2.69) (layer "F.Cu") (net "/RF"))
 (segment (start 35.35 33) (end 35.8 34.1) (width 7.34) (layer "F.Cu") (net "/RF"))
 (segment (start 34.585 27.75) (end 34.585 28) (width 1.32) (layer "F.Cu") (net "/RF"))
 (segment (start 34.585 26.5) (end 34.585 26.8) (width 1.39) (layer "F.Cu") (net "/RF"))
 (segment (start 34.585 30.35) (end 34.585 30.9) (width 4.02) (layer "F.Cu") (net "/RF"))
 (segment (start 35.95 24.8125) (end 36.3 24.8125) (width 1.53) (layer "F.Cu") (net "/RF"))
 (segment (start 34.585 26.8) (end 34.585 27.05) (width 1.3) (layer "F.Cu") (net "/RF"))
 (segment (start 34.585 28.65) (end 34.585 29) (width 1.88) (layer "F.Cu") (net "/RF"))
 (segment (start 35.1 24.8125) (end 35.55 24.8125) (width 2.17) (layer "F.Cu") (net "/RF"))
 (segment (start 34.585 27.25) (end 34.585 27.5) (width 1.26) (layer "F.Cu") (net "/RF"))
 (segment (start 34.585 29.85) (end 34.585 30.35) (width 3.29) (layer "F.Cu") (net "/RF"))
 (segment (start 37.85 24.8125) (end 38.3 24.8125) (width 1.46) (layer "F.Cu") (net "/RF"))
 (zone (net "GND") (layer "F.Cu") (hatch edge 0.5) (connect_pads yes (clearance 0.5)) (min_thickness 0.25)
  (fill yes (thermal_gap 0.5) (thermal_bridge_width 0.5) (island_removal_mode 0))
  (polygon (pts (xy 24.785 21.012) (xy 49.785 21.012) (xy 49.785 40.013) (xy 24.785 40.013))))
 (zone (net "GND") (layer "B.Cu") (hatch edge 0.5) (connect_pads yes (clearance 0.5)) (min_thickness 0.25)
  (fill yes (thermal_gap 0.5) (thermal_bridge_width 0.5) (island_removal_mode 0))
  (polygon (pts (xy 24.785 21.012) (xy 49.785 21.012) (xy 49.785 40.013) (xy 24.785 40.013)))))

